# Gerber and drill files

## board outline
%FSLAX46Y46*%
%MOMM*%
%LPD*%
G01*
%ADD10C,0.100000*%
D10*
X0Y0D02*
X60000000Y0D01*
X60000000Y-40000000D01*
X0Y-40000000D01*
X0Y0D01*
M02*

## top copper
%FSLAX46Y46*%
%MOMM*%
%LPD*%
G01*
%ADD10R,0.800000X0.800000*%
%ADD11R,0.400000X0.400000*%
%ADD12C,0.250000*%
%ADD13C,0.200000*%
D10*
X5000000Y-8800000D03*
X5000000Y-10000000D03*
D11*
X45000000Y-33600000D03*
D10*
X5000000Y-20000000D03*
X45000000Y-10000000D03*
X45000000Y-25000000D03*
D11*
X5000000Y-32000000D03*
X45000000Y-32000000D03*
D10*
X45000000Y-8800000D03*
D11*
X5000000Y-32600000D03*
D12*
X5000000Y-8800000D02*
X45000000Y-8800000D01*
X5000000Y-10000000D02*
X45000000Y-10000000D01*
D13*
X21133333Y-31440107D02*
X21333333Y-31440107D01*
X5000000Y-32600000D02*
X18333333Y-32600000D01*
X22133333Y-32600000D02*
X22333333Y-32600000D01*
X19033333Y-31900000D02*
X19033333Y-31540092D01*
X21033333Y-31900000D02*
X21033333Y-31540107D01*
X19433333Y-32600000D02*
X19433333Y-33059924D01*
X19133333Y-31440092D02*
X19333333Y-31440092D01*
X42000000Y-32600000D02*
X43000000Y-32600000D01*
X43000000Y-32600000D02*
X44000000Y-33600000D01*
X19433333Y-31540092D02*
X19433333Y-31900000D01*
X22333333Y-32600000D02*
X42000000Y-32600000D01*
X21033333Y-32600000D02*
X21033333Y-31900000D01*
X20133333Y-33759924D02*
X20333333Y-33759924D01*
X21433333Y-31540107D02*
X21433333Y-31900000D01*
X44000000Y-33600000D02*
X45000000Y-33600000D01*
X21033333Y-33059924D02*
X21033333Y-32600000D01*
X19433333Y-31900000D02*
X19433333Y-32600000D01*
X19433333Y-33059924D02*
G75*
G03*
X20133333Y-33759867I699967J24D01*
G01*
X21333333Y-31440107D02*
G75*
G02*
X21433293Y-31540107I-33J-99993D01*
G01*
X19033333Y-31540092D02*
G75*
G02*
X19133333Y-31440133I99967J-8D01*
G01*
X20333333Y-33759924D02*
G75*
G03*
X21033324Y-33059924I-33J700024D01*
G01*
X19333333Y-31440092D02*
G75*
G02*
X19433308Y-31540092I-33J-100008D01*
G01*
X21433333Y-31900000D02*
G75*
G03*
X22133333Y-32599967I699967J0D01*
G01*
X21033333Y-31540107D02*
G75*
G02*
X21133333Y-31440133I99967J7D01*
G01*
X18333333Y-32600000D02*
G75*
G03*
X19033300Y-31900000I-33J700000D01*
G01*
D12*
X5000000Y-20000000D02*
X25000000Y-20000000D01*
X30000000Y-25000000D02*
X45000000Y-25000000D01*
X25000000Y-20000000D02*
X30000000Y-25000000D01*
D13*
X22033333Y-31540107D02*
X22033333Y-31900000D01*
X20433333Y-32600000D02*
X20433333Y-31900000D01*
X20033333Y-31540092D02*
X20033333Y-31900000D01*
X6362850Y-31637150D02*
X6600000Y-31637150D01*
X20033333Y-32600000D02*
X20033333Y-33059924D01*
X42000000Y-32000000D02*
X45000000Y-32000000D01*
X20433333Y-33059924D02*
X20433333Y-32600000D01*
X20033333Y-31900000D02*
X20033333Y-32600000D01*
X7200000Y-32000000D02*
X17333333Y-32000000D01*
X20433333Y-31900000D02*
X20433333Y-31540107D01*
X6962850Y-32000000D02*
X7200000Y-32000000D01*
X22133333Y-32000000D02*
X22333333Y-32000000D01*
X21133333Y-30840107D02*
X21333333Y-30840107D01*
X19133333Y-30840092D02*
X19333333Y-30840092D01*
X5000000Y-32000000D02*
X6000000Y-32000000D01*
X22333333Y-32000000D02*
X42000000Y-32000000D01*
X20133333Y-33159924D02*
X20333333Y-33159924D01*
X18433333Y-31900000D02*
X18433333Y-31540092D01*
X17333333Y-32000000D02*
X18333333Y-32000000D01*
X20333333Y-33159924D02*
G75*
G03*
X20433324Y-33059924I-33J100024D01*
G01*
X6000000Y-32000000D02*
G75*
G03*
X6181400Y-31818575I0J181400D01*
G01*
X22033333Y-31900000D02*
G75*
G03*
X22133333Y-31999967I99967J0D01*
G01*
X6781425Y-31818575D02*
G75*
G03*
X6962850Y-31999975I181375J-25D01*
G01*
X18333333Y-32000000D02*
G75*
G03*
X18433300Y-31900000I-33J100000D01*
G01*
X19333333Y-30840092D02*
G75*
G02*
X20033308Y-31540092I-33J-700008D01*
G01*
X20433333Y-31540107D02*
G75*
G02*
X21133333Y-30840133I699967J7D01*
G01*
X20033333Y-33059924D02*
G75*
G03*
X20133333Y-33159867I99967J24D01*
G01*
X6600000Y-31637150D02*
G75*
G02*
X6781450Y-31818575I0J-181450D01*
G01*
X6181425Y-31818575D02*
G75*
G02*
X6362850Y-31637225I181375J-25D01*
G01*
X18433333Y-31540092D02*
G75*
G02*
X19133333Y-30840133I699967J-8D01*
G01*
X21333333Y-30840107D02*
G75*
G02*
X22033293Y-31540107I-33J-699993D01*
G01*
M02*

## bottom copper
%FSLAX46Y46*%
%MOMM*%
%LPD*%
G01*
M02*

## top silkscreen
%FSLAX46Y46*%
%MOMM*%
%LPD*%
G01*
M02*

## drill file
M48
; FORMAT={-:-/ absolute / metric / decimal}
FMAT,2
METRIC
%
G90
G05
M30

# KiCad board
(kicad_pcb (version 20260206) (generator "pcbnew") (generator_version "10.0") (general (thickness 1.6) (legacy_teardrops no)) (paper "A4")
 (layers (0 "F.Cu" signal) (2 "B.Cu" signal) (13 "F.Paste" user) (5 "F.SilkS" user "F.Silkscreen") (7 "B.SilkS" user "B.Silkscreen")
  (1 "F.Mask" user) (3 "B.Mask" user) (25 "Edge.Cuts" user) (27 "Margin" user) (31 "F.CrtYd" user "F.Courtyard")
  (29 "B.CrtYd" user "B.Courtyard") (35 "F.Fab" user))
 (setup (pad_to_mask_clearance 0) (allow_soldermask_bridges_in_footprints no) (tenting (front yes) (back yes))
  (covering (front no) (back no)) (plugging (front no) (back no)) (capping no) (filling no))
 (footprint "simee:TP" (layer "F.Cu") (at 5 8.8)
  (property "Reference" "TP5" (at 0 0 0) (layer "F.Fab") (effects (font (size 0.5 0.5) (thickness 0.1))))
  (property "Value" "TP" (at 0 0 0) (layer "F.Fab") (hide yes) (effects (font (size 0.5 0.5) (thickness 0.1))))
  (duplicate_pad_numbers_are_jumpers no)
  (pad "1" smd rect (at 0 0) (size 0.8 0.8) (layers "F.Cu" "F.Mask") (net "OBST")))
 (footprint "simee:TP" (layer "F.Cu") (at 5 10)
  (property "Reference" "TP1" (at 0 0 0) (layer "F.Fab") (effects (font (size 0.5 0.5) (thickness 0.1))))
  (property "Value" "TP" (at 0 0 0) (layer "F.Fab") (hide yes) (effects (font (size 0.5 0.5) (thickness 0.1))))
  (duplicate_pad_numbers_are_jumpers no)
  (pad "1" smd rect (at 0 0) (size 0.8 0.8) (layers "F.Cu" "F.Mask") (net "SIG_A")))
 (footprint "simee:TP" (layer "F.Cu") (at 45 33.6)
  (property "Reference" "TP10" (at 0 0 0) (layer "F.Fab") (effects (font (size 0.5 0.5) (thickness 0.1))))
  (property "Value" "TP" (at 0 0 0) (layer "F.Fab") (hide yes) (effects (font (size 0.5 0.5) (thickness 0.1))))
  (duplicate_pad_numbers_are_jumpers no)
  (pad "1" smd rect (at 0 0) (size 0.4 0.4) (layers "F.Cu" "F.Mask") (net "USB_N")))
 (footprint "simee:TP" (layer "F.Cu") (at 5 20)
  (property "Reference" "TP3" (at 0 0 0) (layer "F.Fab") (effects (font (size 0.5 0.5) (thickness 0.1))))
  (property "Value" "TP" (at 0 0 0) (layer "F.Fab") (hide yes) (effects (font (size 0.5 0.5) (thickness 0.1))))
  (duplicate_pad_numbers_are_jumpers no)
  (pad "1" smd rect (at 0 0) (size 0.8 0.8) (layers "F.Cu" "F.Mask") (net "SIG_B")))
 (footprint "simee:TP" (layer "F.Cu") (at 45 10)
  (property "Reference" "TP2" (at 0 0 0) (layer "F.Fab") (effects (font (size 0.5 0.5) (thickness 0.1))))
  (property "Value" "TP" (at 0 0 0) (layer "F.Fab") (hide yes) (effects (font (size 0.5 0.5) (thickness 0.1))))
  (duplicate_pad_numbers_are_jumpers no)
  (pad "1" smd rect (at 0 0) (size 0.8 0.8) (layers "F.Cu" "F.Mask") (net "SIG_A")))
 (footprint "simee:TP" (layer "F.Cu") (at 45 25)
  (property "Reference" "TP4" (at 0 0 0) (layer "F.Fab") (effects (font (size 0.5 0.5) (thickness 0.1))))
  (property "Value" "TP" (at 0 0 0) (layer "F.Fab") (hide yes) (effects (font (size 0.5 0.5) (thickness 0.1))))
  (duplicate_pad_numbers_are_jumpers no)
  (pad "1" smd rect (at 0 0) (size 0.8 0.8) (layers "F.Cu" "F.Mask") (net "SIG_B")))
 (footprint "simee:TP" (layer "F.Cu") (at 5 32)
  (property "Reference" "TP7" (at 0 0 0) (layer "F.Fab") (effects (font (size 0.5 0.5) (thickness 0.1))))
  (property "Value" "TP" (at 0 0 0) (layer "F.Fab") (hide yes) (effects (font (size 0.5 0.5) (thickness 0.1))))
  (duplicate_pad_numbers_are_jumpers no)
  (pad "1" smd rect (at 0 0) (size 0.4 0.4) (layers "F.Cu" "F.Mask") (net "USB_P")))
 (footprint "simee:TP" (layer "F.Cu") (at 45 32)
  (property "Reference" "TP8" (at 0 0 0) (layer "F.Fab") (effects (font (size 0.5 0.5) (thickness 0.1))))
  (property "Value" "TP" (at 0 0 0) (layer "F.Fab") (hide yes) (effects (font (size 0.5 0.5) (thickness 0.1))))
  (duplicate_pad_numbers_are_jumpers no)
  (pad "1" smd rect (at 0 0) (size 0.4 0.4) (layers "F.Cu" "F.Mask") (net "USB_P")))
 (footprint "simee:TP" (layer "F.Cu") (at 45 8.8)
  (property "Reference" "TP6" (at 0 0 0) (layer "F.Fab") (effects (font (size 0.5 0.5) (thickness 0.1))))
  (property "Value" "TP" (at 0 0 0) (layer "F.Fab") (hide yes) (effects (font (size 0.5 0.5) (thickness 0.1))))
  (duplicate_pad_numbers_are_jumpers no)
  (pad "1" smd rect (at 0 0) (size 0.8 0.8) (layers "F.Cu" "F.Mask") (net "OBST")))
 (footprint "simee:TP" (layer "F.Cu") (at 5 32.6)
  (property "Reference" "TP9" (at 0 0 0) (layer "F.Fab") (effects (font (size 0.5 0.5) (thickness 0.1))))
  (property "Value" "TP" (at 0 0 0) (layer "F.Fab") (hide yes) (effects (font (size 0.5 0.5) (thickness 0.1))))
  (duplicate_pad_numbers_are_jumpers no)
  (pad "1" smd rect (at 0 0) (size 0.4 0.4) (layers "F.Cu" "F.Mask") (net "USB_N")))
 (gr_rect (start 0 0) (end 60 40) (stroke (width 0.1) (type default)) (fill no) (layer "Edge.Cuts"))
 (segment (start 5 8.8) (end 45 8.8) (width 0.25) (layer "F.Cu") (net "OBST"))
 (segment (start 5 10) (end 45 10) (width 0.25) (layer "F.Cu") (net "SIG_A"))
 (segment (start 21.133333 31.440107) (end 21.333333 31.440107) (width 0.2) (layer "F.Cu") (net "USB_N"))
 (segment (start 5 32.6) (end 18.333333 32.6) (width 0.2) (layer "F.Cu") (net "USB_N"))
 (segment (start 22.133333 32.6) (end 22.333333 32.6) (width 0.2) (layer "F.Cu") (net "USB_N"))
 (segment (start 19.033333 31.9) (end 19.033333 31.540092) (width 0.2) (layer "F.Cu") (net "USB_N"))
 (segment (start 21.033333 31.9) (end 21.033333 31.540107) (width 0.2) (layer "F.Cu") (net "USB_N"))
 (segment (start 19.433333 32.6) (end 19.433333 33.059924) (width 0.2) (layer "F.Cu") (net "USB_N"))
 (segment (start 19.133333 31.440092) (end 19.333333 31.440092) (width 0.2) (layer "F.Cu") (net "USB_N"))
 (segment (start 42 32.6) (end 43 32.6) (width 0.2) (layer "F.Cu") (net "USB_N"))
 (segment (start 43 32.6) (end 44 33.6) (width 0.2) (layer "F.Cu") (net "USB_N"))
 (segment (start 19.433333 31.540092) (end 19.433333 31.9) (width 0.2) (layer "F.Cu") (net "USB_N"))
 (segment (start 22.333333 32.6) (end 42 32.6) (width 0.2) (layer "F.Cu") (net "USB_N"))
 (segment (start 21.033333 32.6) (end 21.033333 31.9) (width 0.2) (layer "F.Cu") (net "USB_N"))
 (segment (start 20.133333 33.759924) (end 20.333333 33.759924) (width 0.2) (layer "F.Cu") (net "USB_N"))
 (segment (start 21.433333 31.540107) (end 21.433333 31.9) (width 0.2) (layer "F.Cu") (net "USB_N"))
 (segment (start 44 33.6) (end 45 33.6) (width 0.2) (layer "F.Cu") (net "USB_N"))
 (segment (start 21.033333 33.059924) (end 21.033333 32.6) (width 0.2) (layer "F.Cu") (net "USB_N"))
 (segment (start 19.433333 31.9) (end 19.433333 32.6) (width 0.2) (layer "F.Cu") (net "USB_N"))
 (arc (start 19.433333 33.059924) (mid 19.638358 33.554899) (end 20.133333 33.759924) (width 0.2) (layer "F.Cu") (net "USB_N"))
 (arc (start 21.333333 31.440107) (mid 21.404044 31.469396) (end 21.433333 31.540107) (width 0.2) (layer "F.Cu") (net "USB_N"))
 (arc (start 19.033333 31.540092) (mid 19.062622 31.469381) (end 19.133333 31.440092) (width 0.2) (layer "F.Cu") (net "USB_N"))
 (arc (start 20.333333 33.759924) (mid 20.828308 33.554899) (end 21.033333 33.059924) (width 0.2) (layer "F.Cu") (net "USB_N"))
 (arc (start 19.333333 31.440092) (mid 19.404044 31.469381) (end 19.433333 31.540092) (width 0.2) (layer "F.Cu") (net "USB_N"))
 (arc (start 21.433333 31.9) (mid 21.638358 32.394975) (end 22.133333 32.6) (width 0.2) (layer "F.Cu") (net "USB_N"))
 (arc (start 21.033333 31.540107) (mid 21.062622 31.469396) (end 21.133333 31.440107) (width 0.2) (layer "F.Cu") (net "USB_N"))
 (arc (start 18.333333 32.6) (mid 18.828308 32.394975) (end 19.033333 31.9) (width 0.2) (layer "F.Cu") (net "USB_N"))
 (segment (start 5 20) (end 25 20) (width 0.25) (layer "F.Cu") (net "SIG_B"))
 (segment (start 30 25) (end 45 25) (width 0.25) (layer "F.Cu") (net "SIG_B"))
 (segment (start 25 20) (end 30 25) (width 0.25) (layer "F.Cu") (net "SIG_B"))
 (segment (start 22.033333 31.540107) (end 22.033333 31.9) (width 0.2) (layer "F.Cu") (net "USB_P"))
 (segment (start 20.433333 32.6) (end 20.433333 31.9) (width 0.2) (layer "F.Cu") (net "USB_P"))
 (segment (start 20.033333 31.540092) (end 20.033333 31.9) (width 0.2) (layer "F.Cu") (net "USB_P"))
 (segment (start 6.36285 31.63715) (end 6.6 31.63715) (width 0.2) (layer "F.Cu") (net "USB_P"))
 (segment (start 20.033333 32.6) (end 20.033333 33.059924) (width 0.2) (layer "F.Cu") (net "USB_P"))
 (segment (start 42 32) (end 45 32) (width 0.2) (layer "F.Cu") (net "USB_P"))
 (segment (start 20.433333 33.059924) (end 20.433333 32.6) (width 0.2) (layer "F.Cu") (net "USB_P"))
 (segment (start 20.033333 31.9) (end 20.033333 32.6) (width 0.2) (layer "F.Cu") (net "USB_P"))
 (segment (start 7.2 32) (end 17.333333 32) (width 0.2) (layer "F.Cu") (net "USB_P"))
 (segment (start 20.433333 31.9) (end 20.433333 31.540107) (width 0.2) (layer "F.Cu") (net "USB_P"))
 (segment (start 6.96285 32) (end 7.2 32) (width 0.2) (layer "F.Cu") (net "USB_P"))
 (segment (start 22.133333 32) (end 22.333333 32) (width 0.2) (layer "F.Cu") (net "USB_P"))
 (segment (start 21.133333 30.840107) (end 21.333333 30.840107) (width 0.2) (layer "F.Cu") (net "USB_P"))
 (segment (start 19.133333 30.840092) (end 19.333333 30.840092) (width 0.2) (layer "F.Cu") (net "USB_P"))
 (segment (start 5 32) (end 6 32) (width 0.2) (layer "F.Cu") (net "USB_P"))
 (segment (start 22.333333 32) (end 42 32) (width 0.2) (layer "F.Cu") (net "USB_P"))
 (segment (start 20.133333 33.159924) (end 20.333333 33.159924) (width 0.2) (layer "F.Cu") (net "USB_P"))
 (segment (start 18.433333 31.9) (end 18.433333 31.540092) (width 0.2) (layer "F.Cu") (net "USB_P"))
 (segment (start 17.333333 32) (end 18.333333 32) (width 0.2) (layer "F.Cu") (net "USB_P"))
 (arc (start 20.333333 33.159924) (mid 20.404044 33.130635) (end 20.433333 33.059924) (width 0.2) (layer "F.Cu") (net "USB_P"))
 (arc (start 6 32) (mid 6.128287 31.946862) (end 6.181425 31.818575) (width 0.2) (layer "F.Cu") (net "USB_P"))
 (arc (start 22.033333 31.9) (mid 22.062622 31.970711) (end 22.133333 32) (width 0.2) (layer "F.Cu") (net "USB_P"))
 (arc (start 6.781425 31.818575) (mid 6.834563 31.946862) (end 6.96285 32) (width 0.2) (layer "F.Cu") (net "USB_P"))
 (arc (start 18.333333 32) (mid 18.404044 31.970711) (end 18.433333 31.9) (width 0.2) (layer "F.Cu") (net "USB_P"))
 (arc (start 19.333333 30.840092) (mid 19.828308 31.045117) (end 20.033333 31.540092) (width 0.2) (layer "F.Cu") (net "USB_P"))
 (arc (start 20.433333 31.540107) (mid 20.638358 31.045132) (end 21.133333 30.840107) (width 0.2) (layer "F.Cu") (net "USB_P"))
 (arc (start 20.033333 33.059924) (mid 20.062622 33.130635) (end 20.133333 33.159924) (width 0.2) (layer "F.Cu") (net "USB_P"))
 (arc (start 6.6 31.63715) (mid 6.728287 31.690288) (end 6.781425 31.818575) (width 0.2) (layer "F.Cu") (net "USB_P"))
 (arc (start 6.181425 31.818575) (mid 6.234563 31.690288) (end 6.36285 31.63715) (width 0.2) (layer "F.Cu") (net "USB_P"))
 (arc (start 18.433333 31.540092) (mid 18.638358 31.045117) (end 19.133333 30.840092) (width 0.2) (layer "F.Cu") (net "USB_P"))
 (arc (start 21.333333 30.840107) (mid 21.828308 31.045132) (end 22.033333 31.540107) (width 0.2) (layer "F.Cu") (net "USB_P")))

